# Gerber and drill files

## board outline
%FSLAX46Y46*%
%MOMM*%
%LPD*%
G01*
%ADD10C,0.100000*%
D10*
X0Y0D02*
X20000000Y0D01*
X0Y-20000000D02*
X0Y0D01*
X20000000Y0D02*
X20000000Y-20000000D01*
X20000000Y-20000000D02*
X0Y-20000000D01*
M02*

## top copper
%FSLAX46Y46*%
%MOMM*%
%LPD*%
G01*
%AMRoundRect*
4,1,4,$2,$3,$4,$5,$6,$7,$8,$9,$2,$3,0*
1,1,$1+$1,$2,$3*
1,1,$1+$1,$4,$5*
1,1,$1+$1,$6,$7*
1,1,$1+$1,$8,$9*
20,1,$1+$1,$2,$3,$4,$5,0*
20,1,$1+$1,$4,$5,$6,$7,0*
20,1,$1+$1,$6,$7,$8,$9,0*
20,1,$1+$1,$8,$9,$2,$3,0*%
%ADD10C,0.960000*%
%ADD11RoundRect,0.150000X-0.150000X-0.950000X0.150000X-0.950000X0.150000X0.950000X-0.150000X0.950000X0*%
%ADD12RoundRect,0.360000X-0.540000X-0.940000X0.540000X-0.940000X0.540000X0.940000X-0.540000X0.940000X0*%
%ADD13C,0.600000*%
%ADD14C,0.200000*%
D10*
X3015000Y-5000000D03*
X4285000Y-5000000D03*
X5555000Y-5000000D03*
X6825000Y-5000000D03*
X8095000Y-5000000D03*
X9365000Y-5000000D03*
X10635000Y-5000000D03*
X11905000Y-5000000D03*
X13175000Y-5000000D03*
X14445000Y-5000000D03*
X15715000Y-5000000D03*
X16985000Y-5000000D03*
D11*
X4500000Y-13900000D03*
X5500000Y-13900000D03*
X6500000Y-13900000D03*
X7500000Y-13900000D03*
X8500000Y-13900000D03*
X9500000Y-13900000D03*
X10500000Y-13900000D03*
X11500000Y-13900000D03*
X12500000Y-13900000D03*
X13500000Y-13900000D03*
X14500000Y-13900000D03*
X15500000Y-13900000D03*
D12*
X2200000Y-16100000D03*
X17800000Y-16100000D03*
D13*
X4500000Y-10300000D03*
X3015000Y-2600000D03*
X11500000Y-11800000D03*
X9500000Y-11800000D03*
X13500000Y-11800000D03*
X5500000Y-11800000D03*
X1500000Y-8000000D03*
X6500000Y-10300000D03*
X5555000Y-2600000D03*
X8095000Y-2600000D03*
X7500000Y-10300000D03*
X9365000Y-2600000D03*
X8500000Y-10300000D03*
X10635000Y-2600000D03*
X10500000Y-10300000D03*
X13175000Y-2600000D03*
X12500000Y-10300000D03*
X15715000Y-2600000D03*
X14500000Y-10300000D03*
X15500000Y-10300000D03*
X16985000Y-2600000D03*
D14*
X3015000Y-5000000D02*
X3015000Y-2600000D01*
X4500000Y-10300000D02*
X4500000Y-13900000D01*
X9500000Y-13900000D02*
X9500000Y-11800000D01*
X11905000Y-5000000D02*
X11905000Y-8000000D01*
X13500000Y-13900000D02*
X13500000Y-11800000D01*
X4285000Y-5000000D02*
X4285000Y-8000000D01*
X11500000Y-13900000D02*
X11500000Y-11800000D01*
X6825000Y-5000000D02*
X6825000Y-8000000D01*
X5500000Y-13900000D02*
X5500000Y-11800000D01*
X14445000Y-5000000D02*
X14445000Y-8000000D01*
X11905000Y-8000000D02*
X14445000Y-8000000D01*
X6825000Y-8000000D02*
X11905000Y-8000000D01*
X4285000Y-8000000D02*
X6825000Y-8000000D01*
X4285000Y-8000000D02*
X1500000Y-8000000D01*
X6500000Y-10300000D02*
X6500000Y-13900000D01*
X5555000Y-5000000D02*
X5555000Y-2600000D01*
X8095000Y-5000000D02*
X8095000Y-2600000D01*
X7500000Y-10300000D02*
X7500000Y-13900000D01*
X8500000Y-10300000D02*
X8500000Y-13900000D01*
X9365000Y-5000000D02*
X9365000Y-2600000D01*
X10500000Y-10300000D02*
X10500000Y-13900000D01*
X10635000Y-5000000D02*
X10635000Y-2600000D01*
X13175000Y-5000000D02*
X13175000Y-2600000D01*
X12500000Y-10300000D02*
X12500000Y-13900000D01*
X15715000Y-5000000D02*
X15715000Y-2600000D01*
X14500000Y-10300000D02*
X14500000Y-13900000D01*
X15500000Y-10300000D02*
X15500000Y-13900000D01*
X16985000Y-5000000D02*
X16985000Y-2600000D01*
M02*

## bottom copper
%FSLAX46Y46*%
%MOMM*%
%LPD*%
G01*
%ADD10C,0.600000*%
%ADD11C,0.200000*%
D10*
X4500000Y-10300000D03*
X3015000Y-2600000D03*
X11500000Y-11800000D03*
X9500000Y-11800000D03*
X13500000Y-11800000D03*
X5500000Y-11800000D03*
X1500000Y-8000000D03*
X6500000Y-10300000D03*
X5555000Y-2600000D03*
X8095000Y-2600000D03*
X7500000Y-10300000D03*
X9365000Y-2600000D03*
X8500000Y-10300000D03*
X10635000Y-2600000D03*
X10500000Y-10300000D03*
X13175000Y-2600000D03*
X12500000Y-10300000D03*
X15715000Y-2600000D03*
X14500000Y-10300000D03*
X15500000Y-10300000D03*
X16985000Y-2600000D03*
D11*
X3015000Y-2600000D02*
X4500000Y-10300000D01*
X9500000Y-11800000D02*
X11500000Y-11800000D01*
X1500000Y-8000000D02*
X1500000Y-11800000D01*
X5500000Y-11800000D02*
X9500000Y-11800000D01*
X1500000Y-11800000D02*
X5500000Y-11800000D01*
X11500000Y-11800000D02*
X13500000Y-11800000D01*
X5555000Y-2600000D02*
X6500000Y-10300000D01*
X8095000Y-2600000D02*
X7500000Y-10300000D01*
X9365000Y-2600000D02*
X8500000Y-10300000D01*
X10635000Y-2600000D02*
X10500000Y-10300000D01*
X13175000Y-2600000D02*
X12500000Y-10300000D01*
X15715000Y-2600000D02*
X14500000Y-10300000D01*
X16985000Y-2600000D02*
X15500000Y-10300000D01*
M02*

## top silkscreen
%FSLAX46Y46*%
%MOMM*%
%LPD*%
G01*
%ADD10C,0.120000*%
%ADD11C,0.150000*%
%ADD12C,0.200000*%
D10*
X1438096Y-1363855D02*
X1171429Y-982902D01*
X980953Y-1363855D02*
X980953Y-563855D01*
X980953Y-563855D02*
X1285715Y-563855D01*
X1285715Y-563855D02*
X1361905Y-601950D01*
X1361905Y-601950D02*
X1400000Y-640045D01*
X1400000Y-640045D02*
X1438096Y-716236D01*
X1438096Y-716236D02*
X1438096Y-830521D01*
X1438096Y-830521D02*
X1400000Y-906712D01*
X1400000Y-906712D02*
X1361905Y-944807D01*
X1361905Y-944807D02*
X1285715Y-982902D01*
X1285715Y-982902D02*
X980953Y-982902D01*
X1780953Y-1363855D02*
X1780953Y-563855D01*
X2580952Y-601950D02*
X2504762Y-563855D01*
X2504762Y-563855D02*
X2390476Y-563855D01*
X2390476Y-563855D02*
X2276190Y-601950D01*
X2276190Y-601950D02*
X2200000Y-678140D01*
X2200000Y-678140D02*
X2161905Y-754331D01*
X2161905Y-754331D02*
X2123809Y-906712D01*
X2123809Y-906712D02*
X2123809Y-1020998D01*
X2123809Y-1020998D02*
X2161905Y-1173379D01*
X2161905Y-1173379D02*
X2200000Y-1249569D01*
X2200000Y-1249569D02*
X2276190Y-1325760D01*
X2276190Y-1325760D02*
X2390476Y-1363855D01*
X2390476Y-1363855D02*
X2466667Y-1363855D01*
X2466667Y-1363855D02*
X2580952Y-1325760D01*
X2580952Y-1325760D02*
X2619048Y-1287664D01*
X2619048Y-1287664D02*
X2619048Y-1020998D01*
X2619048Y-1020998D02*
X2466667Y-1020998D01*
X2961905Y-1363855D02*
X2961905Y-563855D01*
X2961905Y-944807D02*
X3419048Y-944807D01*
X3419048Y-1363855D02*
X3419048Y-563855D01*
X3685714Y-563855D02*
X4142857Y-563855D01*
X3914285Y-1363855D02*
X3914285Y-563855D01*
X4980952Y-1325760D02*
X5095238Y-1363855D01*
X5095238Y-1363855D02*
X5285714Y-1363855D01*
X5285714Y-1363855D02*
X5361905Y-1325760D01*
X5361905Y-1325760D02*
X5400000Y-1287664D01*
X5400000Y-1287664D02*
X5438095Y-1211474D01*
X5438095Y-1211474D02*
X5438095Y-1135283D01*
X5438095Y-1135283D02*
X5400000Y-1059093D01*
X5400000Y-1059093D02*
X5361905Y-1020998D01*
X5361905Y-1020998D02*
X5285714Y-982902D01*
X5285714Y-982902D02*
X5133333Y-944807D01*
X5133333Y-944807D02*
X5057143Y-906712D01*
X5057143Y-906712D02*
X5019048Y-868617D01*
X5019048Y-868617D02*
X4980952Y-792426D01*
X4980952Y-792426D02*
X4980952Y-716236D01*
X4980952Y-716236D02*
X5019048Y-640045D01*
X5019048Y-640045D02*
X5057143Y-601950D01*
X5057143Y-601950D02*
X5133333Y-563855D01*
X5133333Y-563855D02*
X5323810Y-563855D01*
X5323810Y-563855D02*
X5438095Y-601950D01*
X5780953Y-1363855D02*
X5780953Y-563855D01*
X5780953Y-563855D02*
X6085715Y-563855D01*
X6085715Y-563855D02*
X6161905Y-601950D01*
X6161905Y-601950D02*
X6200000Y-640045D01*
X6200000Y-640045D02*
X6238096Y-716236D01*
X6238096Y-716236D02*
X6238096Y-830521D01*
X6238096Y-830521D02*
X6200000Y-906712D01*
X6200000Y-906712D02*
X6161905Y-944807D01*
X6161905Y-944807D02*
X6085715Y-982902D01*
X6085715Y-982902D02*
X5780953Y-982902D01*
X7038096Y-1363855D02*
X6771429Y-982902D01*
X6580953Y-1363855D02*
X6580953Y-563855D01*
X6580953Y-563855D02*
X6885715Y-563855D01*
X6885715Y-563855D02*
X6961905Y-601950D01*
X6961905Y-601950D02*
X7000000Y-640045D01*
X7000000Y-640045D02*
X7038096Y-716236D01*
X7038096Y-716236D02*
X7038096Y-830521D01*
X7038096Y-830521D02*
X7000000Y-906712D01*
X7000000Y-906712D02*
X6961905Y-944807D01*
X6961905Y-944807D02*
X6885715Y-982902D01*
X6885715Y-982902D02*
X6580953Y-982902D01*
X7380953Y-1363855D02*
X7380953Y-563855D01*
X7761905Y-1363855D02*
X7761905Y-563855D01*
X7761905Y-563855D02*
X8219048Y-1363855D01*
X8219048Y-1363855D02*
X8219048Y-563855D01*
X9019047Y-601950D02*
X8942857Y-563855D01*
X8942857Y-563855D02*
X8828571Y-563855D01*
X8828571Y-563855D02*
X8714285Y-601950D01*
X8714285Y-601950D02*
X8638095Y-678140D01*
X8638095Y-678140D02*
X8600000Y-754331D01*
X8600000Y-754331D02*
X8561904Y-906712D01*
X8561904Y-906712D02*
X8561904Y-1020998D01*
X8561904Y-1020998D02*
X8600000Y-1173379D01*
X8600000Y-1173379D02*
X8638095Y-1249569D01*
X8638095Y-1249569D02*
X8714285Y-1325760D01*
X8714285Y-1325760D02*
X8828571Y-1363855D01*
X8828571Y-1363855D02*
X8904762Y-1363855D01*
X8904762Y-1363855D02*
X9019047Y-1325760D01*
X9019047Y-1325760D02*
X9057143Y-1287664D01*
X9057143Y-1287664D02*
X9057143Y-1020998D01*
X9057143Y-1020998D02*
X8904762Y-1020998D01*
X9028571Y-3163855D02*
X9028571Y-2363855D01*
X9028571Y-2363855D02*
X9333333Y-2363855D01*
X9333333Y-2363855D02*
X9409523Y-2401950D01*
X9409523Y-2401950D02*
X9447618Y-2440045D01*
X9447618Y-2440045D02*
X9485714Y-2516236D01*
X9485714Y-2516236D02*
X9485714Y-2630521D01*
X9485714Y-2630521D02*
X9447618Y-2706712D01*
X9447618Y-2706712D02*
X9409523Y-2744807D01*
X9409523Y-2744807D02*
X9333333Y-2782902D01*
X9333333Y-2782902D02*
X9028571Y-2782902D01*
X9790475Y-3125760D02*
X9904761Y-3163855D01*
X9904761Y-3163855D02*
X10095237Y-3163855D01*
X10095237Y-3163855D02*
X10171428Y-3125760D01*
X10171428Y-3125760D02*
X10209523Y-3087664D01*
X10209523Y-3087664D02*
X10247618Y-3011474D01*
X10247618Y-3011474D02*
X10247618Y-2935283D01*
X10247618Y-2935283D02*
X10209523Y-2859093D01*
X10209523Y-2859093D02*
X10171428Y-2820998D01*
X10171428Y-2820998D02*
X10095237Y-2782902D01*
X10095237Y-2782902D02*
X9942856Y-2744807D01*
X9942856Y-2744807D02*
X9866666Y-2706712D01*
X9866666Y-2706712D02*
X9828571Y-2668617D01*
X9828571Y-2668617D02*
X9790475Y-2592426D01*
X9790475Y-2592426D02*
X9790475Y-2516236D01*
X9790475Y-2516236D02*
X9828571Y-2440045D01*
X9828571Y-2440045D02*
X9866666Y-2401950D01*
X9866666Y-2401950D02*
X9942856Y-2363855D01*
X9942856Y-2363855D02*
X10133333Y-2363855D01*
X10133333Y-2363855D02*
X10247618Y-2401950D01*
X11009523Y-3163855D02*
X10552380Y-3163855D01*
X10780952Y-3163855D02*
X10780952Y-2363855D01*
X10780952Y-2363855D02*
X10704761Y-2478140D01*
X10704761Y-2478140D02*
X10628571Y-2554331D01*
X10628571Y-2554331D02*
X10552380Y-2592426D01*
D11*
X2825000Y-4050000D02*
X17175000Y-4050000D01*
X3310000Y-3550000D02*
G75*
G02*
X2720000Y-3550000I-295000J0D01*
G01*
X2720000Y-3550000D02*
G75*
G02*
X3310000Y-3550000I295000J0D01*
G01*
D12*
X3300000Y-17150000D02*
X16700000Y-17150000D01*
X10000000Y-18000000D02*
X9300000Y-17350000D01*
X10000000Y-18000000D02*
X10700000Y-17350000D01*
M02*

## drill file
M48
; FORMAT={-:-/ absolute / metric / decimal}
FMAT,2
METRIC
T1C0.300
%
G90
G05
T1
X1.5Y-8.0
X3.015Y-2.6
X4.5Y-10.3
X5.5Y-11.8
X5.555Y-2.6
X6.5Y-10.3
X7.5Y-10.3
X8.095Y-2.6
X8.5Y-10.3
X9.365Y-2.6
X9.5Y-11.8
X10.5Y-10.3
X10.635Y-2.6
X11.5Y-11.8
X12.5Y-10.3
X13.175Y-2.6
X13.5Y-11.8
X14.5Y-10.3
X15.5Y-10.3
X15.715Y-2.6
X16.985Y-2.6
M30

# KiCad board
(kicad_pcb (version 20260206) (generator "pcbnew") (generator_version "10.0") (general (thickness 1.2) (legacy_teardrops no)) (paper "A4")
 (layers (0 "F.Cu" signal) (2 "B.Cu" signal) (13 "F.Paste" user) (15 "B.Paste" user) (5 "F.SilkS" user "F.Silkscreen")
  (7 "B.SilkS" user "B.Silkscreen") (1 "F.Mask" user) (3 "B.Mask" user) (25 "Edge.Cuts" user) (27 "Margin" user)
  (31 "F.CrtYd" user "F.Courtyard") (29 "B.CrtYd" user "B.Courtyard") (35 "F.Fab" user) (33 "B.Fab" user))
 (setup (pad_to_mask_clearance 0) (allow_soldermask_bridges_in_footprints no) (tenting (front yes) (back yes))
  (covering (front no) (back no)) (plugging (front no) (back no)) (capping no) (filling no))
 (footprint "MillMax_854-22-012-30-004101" (layer "F.Cu") (at 10 5)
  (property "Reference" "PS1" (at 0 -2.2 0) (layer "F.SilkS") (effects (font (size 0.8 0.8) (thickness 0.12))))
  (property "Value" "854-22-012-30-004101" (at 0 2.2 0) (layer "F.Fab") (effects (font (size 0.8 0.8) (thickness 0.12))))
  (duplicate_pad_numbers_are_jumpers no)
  (fp_line (start -7.175 -0.95) (end 7.175 -0.95) (stroke (width 0.15) (type solid)) (layer "F.SilkS"))
  (fp_circle (center -6.985 -1.45) (end -6.69 -1.45) (stroke (width 0.15) (type solid)) (fill no) (layer "F.SilkS"))
  (pad "1" smd circle (at -6.985 0) (size 0.96 0.96) (layers "F.Cu" "F.Mask" "F.Paste") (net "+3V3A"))
  (pad "2" smd circle (at -5.715 0) (size 0.96 0.96) (layers "F.Cu" "F.Mask" "F.Paste") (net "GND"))
  (pad "3" smd circle (at -4.445 0) (size 0.96 0.96) (layers "F.Cu" "F.Mask" "F.Paste") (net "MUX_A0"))
  (pad "4" smd circle (at -3.175 0) (size 0.96 0.96) (layers "F.Cu" "F.Mask" "F.Paste") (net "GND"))
  (pad "5" smd circle (at -1.905 0) (size 0.96 0.96) (layers "F.Cu" "F.Mask" "F.Paste") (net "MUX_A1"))
  (pad "6" smd circle (at -0.635 0) (size 0.96 0.96) (layers "F.Cu" "F.Mask" "F.Paste") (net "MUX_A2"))
  (pad "7" smd circle (at 0.635 0) (size 0.96 0.96) (layers "F.Cu" "F.Mask" "F.Paste") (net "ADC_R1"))
  (pad "8" smd circle (at 1.905 0) (size 0.96 0.96) (layers "F.Cu" "F.Mask" "F.Paste") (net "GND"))
  (pad "9" smd circle (at 3.175 0) (size 0.96 0.96) (layers "F.Cu" "F.Mask" "F.Paste") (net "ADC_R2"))
  (pad "10" smd circle (at 4.445 0) (size 0.96 0.96) (layers "F.Cu" "F.Mask" "F.Paste") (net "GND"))
  (pad "11" smd circle (at 5.715 0) (size 0.96 0.96) (layers "F.Cu" "F.Mask" "F.Paste") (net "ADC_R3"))
  (pad "12" smd circle (at 6.985 0) (size 0.96 0.96) (layers "F.Cu" "F.Mask" "F.Paste") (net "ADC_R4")))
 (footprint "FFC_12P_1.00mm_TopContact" (layer "F.Cu") (at 10 15)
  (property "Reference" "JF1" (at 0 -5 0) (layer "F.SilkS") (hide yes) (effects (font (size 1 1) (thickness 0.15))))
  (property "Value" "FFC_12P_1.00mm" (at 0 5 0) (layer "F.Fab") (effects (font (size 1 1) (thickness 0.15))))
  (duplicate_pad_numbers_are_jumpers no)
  (fp_line (start -6.7 2.15) (end 6.7 2.15) (stroke (width 0.2) (type solid)) (layer "F.SilkS"))
  (fp_line (start 0 3) (end -0.7 2.35) (stroke (width 0.2) (type solid)) (layer "F.SilkS"))
  (fp_line (start 0 3) (end 0.7 2.35) (stroke (width 0.2) (type solid)) (layer "F.SilkS"))
  (pad "1" smd roundrect (at -5.5 -1.1) (size 0.6 2.2) (layers "F.Cu" "F.Mask" "F.Paste") (roundrect_rratio 0.25) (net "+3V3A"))
  (pad "2" smd roundrect (at -4.5 -1.1) (size 0.6 2.2) (layers "F.Cu" "F.Mask" "F.Paste") (roundrect_rratio 0.25) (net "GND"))
  (pad "3" smd roundrect (at -3.5 -1.1) (size 0.6 2.2) (layers "F.Cu" "F.Mask" "F.Paste") (roundrect_rratio 0.25) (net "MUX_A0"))
  (pad "4" smd roundrect (at -2.5 -1.1) (size 0.6 2.2) (layers "F.Cu" "F.Mask" "F.Paste") (roundrect_rratio 0.25) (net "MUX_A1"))
  (pad "5" smd roundrect (at -1.5 -1.1) (size 0.6 2.2) (layers "F.Cu" "F.Mask" "F.Paste") (roundrect_rratio 0.25) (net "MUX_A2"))
  (pad "6" smd roundrect (at -0.5 -1.1) (size 0.6 2.2) (layers "F.Cu" "F.Mask" "F.Paste") (roundrect_rratio 0.25) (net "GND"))
  (pad "7" smd roundrect (at 0.5 -1.1) (size 0.6 2.2) (layers "F.Cu" "F.Mask" "F.Paste") (roundrect_rratio 0.25) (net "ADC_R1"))
  (pad "8" smd roundrect (at 1.5 -1.1) (size 0.6 2.2) (layers "F.Cu" "F.Mask" "F.Paste") (roundrect_rratio 0.25) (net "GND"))
  (pad "9" smd roundrect (at 2.5 -1.1) (size 0.6 2.2) (layers "F.Cu" "F.Mask" "F.Paste") (roundrect_rratio 0.25) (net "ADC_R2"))
  (pad "10" smd roundrect (at 3.5 -1.1) (size 0.6 2.2) (layers "F.Cu" "F.Mask" "F.Paste") (roundrect_rratio 0.25) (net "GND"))
  (pad "11" smd roundrect (at 4.5 -1.1) (size 0.6 2.2) (layers "F.Cu" "F.Mask" "F.Paste") (roundrect_rratio 0.25) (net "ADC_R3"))
  (pad "12" smd roundrect (at 5.5 -1.1) (size 0.6 2.2) (layers "F.Cu" "F.Mask" "F.Paste") (roundrect_rratio 0.25) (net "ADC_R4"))
  (pad "MP" smd roundrect (at -7.8 1.1) (size 1.8 2.6) (layers "F.Cu" "F.Mask" "F.Paste") (roundrect_rratio 0.2))
  (pad "MP" smd roundrect (at 7.8 1.1) (size 1.8 2.6) (layers "F.Cu" "F.Mask" "F.Paste") (roundrect_rratio 0.2)))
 (gr_line (start 0 0) (end 20 0) (stroke (width 0.1) (type solid)) (layer "Edge.Cuts"))
 (gr_line (start 0 20) (end 0 0) (stroke (width 0.1) (type solid)) (layer "Edge.Cuts"))
 (gr_line (start 20 0) (end 20 20) (stroke (width 0.1) (type solid)) (layer "Edge.Cuts"))
 (gr_line (start 20 20) (end 0 20) (stroke (width 0.1) (type solid)) (layer "Edge.Cuts"))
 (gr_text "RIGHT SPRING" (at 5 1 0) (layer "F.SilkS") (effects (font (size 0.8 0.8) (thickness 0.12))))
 (segment (start 3.015 5) (end 3.015 2.6) (width 0.2) (layer "F.Cu") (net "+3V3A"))
 (segment (start 4.5 10.3) (end 4.5 13.9) (width 0.2) (layer "F.Cu") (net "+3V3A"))
 (via (at 4.5 10.3) (size 0.6) (drill 0.3) (layers "F.Cu" "B.Cu") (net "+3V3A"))
 (via (at 3.015 2.6) (size 0.6) (drill 0.3) (layers "F.Cu" "B.Cu") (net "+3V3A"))
 (segment (start 3.015 2.6) (end 4.5 10.3) (width 0.2) (layer "B.Cu") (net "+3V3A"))
 (segment (start 9.5 13.9) (end 9.5 11.8) (width 0.2) (layer "F.Cu") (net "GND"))
 (segment (start 11.905 5) (end 11.905 8) (width 0.2) (layer "F.Cu") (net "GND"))
 (segment (start 13.5 13.9) (end 13.5 11.8) (width 0.2) (layer "F.Cu") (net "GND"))
 (segment (start 4.285 5) (end 4.285 8) (width 0.2) (layer "F.Cu") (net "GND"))
 (segment (start 11.5 13.9) (end 11.5 11.8) (width 0.2) (layer "F.Cu") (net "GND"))
 (segment (start 6.825 5) (end 6.825 8) (width 0.2) (layer "F.Cu") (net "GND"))
 (segment (start 5.5 13.9) (end 5.5 11.8) (width 0.2) (layer "F.Cu") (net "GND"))
 (segment (start 14.445 5) (end 14.445 8) (width 0.2) (layer "F.Cu") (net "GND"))
 (segment (start 11.905 8) (end 14.445 8) (width 0.2) (layer "F.Cu") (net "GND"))
 (segment (start 6.825 8) (end 11.905 8) (width 0.2) (layer "F.Cu") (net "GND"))
 (segment (start 4.285 8) (end 6.825 8) (width 0.2) (layer "F.Cu") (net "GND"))
 (segment (start 4.285 8) (end 1.5 8) (width 0.2) (layer "F.Cu") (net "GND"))
 (via (at 11.5 11.8) (size 0.6) (drill 0.3) (layers "F.Cu" "B.Cu") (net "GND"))
 (via (at 9.5 11.8) (size 0.6) (drill 0.3) (layers "F.Cu" "B.Cu") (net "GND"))
 (via (at 13.5 11.8) (size 0.6) (drill 0.3) (layers "F.Cu" "B.Cu") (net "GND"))
 (via (at 5.5 11.8) (size 0.6) (drill 0.3) (layers "F.Cu" "B.Cu") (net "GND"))
 (via (at 1.5 8) (size 0.6) (drill 0.3) (layers "F.Cu" "B.Cu") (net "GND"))
 (segment (start 9.5 11.8) (end 11.5 11.8) (width 0.2) (layer "B.Cu") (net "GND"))
 (segment (start 1.5 8) (end 1.5 11.8) (width 0.2) (layer "B.Cu") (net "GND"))
 (segment (start 5.5 11.8) (end 9.5 11.8) (width 0.2) (layer "B.Cu") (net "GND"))
 (segment (start 1.5 11.8) (end 5.5 11.8) (width 0.2) (layer "B.Cu") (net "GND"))
 (segment (start 11.5 11.8) (end 13.5 11.8) (width 0.2) (layer "B.Cu") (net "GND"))
 (segment (start 6.5 10.3) (end 6.5 13.9) (width 0.2) (layer "F.Cu") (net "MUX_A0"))
 (segment (start 5.555 5) (end 5.555 2.6) (width 0.2) (layer "F.Cu") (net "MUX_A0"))
 (via (at 6.5 10.3) (size 0.6) (drill 0.3) (layers "F.Cu" "B.Cu") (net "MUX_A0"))
 (via (at 5.555 2.6) (size 0.6) (drill 0.3) (layers "F.Cu" "B.Cu") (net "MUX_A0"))
 (segment (start 5.555 2.6) (end 6.5 10.3) (width 0.2) (layer "B.Cu") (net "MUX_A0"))
 (segment (start 8.095 5) (end 8.095 2.6) (width 0.2) (layer "F.Cu") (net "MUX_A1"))
 (segment (start 7.5 10.3) (end 7.5 13.9) (width 0.2) (layer "F.Cu") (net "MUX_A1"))
 (via (at 8.095 2.6) (size 0.6) (drill 0.3) (layers "F.Cu" "B.Cu") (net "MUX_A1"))
 (via (at 7.5 10.3) (size 0.6) (drill 0.3) (layers "F.Cu" "B.Cu") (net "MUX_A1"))
 (segment (start 8.095 2.6) (end 7.5 10.3) (width 0.2) (layer "B.Cu") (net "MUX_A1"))
 (segment (start 8.5 10.3) (end 8.5 13.9) (width 0.2) (layer "F.Cu") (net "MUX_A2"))
 (segment (start 9.365 5) (end 9.365 2.6) (width 0.2) (layer "F.Cu") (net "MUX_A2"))
 (via (at 9.365 2.6) (size 0.6) (drill 0.3) (layers "F.Cu" "B.Cu") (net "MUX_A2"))
 (via (at 8.5 10.3) (size 0.6) (drill 0.3) (layers "F.Cu" "B.Cu") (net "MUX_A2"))
 (segment (start 9.365 2.6) (end 8.5 10.3) (width 0.2) (layer "B.Cu") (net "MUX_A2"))
 (segment (start 10.5 10.3) (end 10.5 13.9) (width 0.2) (layer "F.Cu") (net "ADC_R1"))
 (segment (start 10.635 5) (end 10.635 2.6) (width 0.2) (layer "F.Cu") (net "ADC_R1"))
 (via (at 10.635 2.6) (size 0.6) (drill 0.3) (layers "F.Cu" "B.Cu") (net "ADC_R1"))
 (via (at 10.5 10.3) (size 0.6) (drill 0.3) (layers "F.Cu" "B.Cu") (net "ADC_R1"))
 (segment (start 10.635 2.6) (end 10.5 10.3) (width 0.2) (layer "B.Cu") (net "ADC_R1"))
 (segment (start 13.175 5) (end 13.175 2.6) (width 0.2) (layer "F.Cu") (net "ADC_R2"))
 (segment (start 12.5 10.3) (end 12.5 13.9) (width 0.2) (layer "F.Cu") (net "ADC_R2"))
 (via (at 13.175 2.6) (size 0.6) (drill 0.3) (layers "F.Cu" "B.Cu") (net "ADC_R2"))
 (via (at 12.5 10.3) (size 0.6) (drill 0.3) (layers "F.Cu" "B.Cu") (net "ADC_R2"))
 (segment (start 13.175 2.6) (end 12.5 10.3) (width 0.2) (layer "B.Cu") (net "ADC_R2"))
 (segment (start 15.715 5) (end 15.715 2.6) (width 0.2) (layer "F.Cu") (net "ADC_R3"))
 (segment (start 14.5 10.3) (end 14.5 13.9) (width 0.2) (layer "F.Cu") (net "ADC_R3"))
 (via (at 15.715 2.6) (size 0.6) (drill 0.3) (layers "F.Cu" "B.Cu") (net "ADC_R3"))
 (via (at 14.5 10.3) (size 0.6) (drill 0.3) (layers "F.Cu" "B.Cu") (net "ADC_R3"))
 (segment (start 15.715 2.6) (end 14.5 10.3) (width 0.2) (layer "B.Cu") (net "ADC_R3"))
 (segment (start 15.5 10.3) (end 15.5 13.9) (width 0.2) (layer "F.Cu") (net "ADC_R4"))
 (segment (start 16.985 5) (end 16.985 2.6) (width 0.2) (layer "F.Cu") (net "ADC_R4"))
 (via (at 15.5 10.3) (size 0.6) (drill 0.3) (layers "F.Cu" "B.Cu") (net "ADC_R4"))
 (via (at 16.985 2.6) (size 0.6) (drill 0.3) (layers "F.Cu" "B.Cu") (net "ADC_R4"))
 (segment (start 16.985 2.6) (end 15.5 10.3) (width 0.2) (layer "B.Cu") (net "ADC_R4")))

